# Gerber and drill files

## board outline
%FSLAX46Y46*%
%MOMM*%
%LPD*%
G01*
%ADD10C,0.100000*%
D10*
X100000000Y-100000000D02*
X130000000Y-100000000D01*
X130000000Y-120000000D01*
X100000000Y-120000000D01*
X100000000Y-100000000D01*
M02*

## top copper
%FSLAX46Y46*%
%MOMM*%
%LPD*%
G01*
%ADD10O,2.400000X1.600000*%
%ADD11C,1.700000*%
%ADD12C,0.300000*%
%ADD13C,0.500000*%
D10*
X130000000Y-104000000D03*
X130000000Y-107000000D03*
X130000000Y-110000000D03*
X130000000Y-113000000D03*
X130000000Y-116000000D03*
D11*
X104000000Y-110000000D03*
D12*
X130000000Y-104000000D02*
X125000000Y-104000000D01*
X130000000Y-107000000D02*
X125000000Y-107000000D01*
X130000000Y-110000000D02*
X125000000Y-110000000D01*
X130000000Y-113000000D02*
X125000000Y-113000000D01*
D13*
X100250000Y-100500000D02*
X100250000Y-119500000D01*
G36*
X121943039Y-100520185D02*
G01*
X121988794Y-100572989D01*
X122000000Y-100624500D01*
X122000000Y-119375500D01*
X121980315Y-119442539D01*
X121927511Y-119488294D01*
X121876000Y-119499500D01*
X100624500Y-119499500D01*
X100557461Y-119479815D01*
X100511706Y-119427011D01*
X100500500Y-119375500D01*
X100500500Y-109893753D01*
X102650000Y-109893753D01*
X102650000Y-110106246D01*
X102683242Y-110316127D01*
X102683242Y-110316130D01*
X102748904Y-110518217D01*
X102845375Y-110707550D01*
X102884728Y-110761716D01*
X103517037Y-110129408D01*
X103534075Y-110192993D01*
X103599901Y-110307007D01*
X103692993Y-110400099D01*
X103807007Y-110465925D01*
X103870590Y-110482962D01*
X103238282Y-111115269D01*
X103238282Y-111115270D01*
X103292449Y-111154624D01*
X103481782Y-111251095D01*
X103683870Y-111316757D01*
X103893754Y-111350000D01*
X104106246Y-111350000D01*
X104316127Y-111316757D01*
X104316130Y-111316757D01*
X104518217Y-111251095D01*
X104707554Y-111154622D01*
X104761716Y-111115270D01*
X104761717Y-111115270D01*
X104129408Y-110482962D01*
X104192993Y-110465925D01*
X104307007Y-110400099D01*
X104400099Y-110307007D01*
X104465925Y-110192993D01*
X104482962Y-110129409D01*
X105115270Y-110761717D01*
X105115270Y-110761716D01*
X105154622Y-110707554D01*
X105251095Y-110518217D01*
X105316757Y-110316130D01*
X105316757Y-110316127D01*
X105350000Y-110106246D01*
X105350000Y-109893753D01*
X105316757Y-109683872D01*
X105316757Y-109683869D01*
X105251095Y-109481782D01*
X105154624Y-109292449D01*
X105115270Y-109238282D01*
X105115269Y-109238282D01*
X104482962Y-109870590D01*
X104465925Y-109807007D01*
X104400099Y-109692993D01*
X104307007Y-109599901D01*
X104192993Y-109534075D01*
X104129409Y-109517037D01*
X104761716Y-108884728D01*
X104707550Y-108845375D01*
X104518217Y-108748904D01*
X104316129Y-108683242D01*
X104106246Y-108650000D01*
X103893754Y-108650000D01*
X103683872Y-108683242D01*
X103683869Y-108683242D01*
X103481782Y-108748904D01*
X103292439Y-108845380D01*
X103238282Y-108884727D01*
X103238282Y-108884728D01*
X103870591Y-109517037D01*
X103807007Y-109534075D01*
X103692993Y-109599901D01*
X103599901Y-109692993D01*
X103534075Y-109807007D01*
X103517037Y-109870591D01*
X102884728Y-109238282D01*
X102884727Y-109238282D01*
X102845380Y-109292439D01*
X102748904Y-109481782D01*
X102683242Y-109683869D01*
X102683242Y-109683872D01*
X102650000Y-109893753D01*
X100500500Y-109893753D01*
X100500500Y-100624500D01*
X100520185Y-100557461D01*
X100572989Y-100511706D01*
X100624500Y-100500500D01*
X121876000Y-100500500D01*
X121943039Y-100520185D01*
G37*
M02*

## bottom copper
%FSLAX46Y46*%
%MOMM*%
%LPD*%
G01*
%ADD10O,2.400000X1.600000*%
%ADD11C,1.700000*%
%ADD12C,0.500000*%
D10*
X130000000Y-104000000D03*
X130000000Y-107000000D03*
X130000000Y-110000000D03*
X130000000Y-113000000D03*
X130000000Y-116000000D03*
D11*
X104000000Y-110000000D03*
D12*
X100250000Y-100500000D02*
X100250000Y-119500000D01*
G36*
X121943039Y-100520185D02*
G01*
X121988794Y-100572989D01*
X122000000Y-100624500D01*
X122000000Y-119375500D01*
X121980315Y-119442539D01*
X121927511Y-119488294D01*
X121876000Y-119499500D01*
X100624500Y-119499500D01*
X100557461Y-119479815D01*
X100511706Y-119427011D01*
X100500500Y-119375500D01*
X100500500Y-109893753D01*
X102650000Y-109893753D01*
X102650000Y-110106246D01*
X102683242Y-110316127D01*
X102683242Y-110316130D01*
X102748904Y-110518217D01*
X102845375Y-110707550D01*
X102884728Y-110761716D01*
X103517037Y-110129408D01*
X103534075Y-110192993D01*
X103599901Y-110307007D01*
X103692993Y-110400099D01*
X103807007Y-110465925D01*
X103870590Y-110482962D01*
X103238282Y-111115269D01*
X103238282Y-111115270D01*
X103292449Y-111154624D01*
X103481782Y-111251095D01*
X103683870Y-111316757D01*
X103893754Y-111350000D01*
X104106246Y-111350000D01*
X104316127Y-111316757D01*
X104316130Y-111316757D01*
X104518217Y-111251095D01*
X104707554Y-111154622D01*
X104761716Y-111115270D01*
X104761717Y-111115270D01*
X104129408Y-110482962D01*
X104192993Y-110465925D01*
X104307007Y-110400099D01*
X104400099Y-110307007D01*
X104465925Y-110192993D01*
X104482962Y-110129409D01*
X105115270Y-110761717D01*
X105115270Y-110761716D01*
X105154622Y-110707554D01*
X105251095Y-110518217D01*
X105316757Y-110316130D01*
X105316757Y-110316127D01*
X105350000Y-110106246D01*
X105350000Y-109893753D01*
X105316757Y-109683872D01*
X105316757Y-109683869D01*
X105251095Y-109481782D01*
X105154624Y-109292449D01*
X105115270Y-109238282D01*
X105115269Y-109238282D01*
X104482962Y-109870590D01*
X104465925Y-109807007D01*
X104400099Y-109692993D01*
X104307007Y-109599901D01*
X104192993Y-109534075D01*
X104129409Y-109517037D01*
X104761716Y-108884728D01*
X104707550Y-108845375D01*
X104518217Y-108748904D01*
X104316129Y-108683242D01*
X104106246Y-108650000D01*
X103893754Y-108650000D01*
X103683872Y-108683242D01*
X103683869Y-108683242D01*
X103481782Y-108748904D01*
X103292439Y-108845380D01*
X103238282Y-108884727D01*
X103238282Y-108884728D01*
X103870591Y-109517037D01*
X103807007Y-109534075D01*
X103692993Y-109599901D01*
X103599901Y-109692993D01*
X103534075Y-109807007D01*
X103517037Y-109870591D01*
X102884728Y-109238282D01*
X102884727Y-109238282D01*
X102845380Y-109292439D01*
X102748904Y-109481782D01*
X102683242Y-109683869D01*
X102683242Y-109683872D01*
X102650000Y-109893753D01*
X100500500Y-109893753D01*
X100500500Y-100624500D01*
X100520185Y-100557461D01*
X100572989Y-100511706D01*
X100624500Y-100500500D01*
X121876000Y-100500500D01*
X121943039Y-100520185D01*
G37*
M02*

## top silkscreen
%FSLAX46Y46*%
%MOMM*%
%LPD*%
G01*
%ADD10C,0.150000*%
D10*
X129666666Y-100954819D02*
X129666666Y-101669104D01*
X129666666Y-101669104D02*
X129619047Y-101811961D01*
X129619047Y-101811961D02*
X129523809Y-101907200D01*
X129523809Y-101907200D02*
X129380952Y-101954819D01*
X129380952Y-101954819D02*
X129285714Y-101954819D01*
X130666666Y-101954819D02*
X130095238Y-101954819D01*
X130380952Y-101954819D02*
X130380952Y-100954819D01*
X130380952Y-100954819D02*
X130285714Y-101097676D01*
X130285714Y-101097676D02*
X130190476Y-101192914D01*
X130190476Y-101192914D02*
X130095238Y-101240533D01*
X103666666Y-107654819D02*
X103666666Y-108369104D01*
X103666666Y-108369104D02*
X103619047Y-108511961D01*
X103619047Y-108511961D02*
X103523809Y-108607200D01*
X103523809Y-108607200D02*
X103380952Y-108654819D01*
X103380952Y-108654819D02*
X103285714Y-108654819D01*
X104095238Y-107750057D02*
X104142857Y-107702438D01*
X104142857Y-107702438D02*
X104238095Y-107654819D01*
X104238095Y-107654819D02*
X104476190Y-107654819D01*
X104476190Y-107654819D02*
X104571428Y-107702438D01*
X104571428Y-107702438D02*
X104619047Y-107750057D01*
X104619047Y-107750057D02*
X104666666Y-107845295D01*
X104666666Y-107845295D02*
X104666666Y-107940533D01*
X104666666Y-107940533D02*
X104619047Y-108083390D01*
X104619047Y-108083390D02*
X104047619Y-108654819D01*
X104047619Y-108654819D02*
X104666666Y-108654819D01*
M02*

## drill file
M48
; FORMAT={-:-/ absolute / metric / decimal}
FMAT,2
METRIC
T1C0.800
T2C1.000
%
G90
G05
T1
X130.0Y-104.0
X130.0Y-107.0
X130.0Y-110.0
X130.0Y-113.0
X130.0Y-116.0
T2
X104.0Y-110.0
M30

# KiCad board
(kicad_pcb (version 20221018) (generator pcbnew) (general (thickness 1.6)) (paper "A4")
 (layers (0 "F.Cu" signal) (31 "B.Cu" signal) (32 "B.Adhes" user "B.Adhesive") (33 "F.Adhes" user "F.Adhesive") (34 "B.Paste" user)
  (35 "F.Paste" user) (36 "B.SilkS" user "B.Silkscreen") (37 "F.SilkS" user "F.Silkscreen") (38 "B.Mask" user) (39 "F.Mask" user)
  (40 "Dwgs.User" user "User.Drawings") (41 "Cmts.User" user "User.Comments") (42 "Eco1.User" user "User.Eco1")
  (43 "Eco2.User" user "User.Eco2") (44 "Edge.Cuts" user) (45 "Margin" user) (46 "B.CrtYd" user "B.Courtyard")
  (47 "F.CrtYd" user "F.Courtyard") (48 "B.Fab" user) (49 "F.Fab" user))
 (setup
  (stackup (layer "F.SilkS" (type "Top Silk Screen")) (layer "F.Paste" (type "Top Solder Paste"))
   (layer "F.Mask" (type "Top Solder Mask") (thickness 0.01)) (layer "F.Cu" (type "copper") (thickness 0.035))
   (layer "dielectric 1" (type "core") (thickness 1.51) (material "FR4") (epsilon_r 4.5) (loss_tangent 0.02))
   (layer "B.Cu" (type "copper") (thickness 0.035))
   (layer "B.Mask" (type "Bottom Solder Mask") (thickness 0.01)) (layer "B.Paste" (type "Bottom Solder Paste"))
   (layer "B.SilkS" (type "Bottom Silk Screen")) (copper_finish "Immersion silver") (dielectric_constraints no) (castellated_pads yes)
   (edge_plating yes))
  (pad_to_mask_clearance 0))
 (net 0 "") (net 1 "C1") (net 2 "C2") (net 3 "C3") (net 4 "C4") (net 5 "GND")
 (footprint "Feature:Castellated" (layer "F.Cu") (at 130 110)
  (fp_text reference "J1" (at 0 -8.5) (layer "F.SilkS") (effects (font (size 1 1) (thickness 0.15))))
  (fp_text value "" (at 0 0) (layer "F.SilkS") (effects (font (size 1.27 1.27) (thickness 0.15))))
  (pad "1" thru_hole oval (at 0 -6) (size 2.4 1.6) (drill 0.8) (layers "*.Cu" "*.Mask") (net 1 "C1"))
  (pad "2" thru_hole oval (at 0 -3) (size 2.4 1.6) (drill 0.8) (layers "*.Cu" "*.Mask") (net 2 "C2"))
  (pad "3" thru_hole oval (at 0 0) (size 2.4 1.6) (drill 0.8) (layers "*.Cu" "*.Mask") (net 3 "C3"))
  (pad "4" thru_hole oval (at 0 3) (size 2.4 1.6) (drill 0.8) (layers "*.Cu" "*.Mask") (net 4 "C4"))
  (pad "5" thru_hole oval (at 0 6) (size 2.4 1.6) (drill 0.8) (layers "*.Cu" "*.Mask") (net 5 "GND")))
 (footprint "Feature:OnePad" (layer "F.Cu") (at 104 110)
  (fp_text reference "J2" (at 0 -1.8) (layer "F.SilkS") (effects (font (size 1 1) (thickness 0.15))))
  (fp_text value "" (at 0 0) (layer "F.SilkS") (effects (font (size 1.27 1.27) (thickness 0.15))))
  (pad "1" thru_hole circle (at 0 0) (size 1.7 1.7) (drill 1) (layers "*.Cu" "*.Mask") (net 5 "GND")))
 (gr_rect (start 100 100) (end 130 120) (stroke (width 0.1) (type solid)) (fill none) (layer "Edge.Cuts"))
 (segment (start 130 104) (end 125 104) (width 0.3) (layer "F.Cu") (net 1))
 (segment (start 130 107) (end 125 107) (width 0.3) (layer "F.Cu") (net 2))
 (segment (start 130 110) (end 125 110) (width 0.3) (layer "F.Cu") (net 3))
 (segment (start 130 113) (end 125 113) (width 0.3) (layer "F.Cu") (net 4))
 (segment (start 100.25 100.5) (end 100.25 119.5) (width 0.5) (layer "F.Cu") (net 5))
 (segment (start 100.25 100.5) (end 100.25 119.5) (width 0.5) (layer "B.Cu") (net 5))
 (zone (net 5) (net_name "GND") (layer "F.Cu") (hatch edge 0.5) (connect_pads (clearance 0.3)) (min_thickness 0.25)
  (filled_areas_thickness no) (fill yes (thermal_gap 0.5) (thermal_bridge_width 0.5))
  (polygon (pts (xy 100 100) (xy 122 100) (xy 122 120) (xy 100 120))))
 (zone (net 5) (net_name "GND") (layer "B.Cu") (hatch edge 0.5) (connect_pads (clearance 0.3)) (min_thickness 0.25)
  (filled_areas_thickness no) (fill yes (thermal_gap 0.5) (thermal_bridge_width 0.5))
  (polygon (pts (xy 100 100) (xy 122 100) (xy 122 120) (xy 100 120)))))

